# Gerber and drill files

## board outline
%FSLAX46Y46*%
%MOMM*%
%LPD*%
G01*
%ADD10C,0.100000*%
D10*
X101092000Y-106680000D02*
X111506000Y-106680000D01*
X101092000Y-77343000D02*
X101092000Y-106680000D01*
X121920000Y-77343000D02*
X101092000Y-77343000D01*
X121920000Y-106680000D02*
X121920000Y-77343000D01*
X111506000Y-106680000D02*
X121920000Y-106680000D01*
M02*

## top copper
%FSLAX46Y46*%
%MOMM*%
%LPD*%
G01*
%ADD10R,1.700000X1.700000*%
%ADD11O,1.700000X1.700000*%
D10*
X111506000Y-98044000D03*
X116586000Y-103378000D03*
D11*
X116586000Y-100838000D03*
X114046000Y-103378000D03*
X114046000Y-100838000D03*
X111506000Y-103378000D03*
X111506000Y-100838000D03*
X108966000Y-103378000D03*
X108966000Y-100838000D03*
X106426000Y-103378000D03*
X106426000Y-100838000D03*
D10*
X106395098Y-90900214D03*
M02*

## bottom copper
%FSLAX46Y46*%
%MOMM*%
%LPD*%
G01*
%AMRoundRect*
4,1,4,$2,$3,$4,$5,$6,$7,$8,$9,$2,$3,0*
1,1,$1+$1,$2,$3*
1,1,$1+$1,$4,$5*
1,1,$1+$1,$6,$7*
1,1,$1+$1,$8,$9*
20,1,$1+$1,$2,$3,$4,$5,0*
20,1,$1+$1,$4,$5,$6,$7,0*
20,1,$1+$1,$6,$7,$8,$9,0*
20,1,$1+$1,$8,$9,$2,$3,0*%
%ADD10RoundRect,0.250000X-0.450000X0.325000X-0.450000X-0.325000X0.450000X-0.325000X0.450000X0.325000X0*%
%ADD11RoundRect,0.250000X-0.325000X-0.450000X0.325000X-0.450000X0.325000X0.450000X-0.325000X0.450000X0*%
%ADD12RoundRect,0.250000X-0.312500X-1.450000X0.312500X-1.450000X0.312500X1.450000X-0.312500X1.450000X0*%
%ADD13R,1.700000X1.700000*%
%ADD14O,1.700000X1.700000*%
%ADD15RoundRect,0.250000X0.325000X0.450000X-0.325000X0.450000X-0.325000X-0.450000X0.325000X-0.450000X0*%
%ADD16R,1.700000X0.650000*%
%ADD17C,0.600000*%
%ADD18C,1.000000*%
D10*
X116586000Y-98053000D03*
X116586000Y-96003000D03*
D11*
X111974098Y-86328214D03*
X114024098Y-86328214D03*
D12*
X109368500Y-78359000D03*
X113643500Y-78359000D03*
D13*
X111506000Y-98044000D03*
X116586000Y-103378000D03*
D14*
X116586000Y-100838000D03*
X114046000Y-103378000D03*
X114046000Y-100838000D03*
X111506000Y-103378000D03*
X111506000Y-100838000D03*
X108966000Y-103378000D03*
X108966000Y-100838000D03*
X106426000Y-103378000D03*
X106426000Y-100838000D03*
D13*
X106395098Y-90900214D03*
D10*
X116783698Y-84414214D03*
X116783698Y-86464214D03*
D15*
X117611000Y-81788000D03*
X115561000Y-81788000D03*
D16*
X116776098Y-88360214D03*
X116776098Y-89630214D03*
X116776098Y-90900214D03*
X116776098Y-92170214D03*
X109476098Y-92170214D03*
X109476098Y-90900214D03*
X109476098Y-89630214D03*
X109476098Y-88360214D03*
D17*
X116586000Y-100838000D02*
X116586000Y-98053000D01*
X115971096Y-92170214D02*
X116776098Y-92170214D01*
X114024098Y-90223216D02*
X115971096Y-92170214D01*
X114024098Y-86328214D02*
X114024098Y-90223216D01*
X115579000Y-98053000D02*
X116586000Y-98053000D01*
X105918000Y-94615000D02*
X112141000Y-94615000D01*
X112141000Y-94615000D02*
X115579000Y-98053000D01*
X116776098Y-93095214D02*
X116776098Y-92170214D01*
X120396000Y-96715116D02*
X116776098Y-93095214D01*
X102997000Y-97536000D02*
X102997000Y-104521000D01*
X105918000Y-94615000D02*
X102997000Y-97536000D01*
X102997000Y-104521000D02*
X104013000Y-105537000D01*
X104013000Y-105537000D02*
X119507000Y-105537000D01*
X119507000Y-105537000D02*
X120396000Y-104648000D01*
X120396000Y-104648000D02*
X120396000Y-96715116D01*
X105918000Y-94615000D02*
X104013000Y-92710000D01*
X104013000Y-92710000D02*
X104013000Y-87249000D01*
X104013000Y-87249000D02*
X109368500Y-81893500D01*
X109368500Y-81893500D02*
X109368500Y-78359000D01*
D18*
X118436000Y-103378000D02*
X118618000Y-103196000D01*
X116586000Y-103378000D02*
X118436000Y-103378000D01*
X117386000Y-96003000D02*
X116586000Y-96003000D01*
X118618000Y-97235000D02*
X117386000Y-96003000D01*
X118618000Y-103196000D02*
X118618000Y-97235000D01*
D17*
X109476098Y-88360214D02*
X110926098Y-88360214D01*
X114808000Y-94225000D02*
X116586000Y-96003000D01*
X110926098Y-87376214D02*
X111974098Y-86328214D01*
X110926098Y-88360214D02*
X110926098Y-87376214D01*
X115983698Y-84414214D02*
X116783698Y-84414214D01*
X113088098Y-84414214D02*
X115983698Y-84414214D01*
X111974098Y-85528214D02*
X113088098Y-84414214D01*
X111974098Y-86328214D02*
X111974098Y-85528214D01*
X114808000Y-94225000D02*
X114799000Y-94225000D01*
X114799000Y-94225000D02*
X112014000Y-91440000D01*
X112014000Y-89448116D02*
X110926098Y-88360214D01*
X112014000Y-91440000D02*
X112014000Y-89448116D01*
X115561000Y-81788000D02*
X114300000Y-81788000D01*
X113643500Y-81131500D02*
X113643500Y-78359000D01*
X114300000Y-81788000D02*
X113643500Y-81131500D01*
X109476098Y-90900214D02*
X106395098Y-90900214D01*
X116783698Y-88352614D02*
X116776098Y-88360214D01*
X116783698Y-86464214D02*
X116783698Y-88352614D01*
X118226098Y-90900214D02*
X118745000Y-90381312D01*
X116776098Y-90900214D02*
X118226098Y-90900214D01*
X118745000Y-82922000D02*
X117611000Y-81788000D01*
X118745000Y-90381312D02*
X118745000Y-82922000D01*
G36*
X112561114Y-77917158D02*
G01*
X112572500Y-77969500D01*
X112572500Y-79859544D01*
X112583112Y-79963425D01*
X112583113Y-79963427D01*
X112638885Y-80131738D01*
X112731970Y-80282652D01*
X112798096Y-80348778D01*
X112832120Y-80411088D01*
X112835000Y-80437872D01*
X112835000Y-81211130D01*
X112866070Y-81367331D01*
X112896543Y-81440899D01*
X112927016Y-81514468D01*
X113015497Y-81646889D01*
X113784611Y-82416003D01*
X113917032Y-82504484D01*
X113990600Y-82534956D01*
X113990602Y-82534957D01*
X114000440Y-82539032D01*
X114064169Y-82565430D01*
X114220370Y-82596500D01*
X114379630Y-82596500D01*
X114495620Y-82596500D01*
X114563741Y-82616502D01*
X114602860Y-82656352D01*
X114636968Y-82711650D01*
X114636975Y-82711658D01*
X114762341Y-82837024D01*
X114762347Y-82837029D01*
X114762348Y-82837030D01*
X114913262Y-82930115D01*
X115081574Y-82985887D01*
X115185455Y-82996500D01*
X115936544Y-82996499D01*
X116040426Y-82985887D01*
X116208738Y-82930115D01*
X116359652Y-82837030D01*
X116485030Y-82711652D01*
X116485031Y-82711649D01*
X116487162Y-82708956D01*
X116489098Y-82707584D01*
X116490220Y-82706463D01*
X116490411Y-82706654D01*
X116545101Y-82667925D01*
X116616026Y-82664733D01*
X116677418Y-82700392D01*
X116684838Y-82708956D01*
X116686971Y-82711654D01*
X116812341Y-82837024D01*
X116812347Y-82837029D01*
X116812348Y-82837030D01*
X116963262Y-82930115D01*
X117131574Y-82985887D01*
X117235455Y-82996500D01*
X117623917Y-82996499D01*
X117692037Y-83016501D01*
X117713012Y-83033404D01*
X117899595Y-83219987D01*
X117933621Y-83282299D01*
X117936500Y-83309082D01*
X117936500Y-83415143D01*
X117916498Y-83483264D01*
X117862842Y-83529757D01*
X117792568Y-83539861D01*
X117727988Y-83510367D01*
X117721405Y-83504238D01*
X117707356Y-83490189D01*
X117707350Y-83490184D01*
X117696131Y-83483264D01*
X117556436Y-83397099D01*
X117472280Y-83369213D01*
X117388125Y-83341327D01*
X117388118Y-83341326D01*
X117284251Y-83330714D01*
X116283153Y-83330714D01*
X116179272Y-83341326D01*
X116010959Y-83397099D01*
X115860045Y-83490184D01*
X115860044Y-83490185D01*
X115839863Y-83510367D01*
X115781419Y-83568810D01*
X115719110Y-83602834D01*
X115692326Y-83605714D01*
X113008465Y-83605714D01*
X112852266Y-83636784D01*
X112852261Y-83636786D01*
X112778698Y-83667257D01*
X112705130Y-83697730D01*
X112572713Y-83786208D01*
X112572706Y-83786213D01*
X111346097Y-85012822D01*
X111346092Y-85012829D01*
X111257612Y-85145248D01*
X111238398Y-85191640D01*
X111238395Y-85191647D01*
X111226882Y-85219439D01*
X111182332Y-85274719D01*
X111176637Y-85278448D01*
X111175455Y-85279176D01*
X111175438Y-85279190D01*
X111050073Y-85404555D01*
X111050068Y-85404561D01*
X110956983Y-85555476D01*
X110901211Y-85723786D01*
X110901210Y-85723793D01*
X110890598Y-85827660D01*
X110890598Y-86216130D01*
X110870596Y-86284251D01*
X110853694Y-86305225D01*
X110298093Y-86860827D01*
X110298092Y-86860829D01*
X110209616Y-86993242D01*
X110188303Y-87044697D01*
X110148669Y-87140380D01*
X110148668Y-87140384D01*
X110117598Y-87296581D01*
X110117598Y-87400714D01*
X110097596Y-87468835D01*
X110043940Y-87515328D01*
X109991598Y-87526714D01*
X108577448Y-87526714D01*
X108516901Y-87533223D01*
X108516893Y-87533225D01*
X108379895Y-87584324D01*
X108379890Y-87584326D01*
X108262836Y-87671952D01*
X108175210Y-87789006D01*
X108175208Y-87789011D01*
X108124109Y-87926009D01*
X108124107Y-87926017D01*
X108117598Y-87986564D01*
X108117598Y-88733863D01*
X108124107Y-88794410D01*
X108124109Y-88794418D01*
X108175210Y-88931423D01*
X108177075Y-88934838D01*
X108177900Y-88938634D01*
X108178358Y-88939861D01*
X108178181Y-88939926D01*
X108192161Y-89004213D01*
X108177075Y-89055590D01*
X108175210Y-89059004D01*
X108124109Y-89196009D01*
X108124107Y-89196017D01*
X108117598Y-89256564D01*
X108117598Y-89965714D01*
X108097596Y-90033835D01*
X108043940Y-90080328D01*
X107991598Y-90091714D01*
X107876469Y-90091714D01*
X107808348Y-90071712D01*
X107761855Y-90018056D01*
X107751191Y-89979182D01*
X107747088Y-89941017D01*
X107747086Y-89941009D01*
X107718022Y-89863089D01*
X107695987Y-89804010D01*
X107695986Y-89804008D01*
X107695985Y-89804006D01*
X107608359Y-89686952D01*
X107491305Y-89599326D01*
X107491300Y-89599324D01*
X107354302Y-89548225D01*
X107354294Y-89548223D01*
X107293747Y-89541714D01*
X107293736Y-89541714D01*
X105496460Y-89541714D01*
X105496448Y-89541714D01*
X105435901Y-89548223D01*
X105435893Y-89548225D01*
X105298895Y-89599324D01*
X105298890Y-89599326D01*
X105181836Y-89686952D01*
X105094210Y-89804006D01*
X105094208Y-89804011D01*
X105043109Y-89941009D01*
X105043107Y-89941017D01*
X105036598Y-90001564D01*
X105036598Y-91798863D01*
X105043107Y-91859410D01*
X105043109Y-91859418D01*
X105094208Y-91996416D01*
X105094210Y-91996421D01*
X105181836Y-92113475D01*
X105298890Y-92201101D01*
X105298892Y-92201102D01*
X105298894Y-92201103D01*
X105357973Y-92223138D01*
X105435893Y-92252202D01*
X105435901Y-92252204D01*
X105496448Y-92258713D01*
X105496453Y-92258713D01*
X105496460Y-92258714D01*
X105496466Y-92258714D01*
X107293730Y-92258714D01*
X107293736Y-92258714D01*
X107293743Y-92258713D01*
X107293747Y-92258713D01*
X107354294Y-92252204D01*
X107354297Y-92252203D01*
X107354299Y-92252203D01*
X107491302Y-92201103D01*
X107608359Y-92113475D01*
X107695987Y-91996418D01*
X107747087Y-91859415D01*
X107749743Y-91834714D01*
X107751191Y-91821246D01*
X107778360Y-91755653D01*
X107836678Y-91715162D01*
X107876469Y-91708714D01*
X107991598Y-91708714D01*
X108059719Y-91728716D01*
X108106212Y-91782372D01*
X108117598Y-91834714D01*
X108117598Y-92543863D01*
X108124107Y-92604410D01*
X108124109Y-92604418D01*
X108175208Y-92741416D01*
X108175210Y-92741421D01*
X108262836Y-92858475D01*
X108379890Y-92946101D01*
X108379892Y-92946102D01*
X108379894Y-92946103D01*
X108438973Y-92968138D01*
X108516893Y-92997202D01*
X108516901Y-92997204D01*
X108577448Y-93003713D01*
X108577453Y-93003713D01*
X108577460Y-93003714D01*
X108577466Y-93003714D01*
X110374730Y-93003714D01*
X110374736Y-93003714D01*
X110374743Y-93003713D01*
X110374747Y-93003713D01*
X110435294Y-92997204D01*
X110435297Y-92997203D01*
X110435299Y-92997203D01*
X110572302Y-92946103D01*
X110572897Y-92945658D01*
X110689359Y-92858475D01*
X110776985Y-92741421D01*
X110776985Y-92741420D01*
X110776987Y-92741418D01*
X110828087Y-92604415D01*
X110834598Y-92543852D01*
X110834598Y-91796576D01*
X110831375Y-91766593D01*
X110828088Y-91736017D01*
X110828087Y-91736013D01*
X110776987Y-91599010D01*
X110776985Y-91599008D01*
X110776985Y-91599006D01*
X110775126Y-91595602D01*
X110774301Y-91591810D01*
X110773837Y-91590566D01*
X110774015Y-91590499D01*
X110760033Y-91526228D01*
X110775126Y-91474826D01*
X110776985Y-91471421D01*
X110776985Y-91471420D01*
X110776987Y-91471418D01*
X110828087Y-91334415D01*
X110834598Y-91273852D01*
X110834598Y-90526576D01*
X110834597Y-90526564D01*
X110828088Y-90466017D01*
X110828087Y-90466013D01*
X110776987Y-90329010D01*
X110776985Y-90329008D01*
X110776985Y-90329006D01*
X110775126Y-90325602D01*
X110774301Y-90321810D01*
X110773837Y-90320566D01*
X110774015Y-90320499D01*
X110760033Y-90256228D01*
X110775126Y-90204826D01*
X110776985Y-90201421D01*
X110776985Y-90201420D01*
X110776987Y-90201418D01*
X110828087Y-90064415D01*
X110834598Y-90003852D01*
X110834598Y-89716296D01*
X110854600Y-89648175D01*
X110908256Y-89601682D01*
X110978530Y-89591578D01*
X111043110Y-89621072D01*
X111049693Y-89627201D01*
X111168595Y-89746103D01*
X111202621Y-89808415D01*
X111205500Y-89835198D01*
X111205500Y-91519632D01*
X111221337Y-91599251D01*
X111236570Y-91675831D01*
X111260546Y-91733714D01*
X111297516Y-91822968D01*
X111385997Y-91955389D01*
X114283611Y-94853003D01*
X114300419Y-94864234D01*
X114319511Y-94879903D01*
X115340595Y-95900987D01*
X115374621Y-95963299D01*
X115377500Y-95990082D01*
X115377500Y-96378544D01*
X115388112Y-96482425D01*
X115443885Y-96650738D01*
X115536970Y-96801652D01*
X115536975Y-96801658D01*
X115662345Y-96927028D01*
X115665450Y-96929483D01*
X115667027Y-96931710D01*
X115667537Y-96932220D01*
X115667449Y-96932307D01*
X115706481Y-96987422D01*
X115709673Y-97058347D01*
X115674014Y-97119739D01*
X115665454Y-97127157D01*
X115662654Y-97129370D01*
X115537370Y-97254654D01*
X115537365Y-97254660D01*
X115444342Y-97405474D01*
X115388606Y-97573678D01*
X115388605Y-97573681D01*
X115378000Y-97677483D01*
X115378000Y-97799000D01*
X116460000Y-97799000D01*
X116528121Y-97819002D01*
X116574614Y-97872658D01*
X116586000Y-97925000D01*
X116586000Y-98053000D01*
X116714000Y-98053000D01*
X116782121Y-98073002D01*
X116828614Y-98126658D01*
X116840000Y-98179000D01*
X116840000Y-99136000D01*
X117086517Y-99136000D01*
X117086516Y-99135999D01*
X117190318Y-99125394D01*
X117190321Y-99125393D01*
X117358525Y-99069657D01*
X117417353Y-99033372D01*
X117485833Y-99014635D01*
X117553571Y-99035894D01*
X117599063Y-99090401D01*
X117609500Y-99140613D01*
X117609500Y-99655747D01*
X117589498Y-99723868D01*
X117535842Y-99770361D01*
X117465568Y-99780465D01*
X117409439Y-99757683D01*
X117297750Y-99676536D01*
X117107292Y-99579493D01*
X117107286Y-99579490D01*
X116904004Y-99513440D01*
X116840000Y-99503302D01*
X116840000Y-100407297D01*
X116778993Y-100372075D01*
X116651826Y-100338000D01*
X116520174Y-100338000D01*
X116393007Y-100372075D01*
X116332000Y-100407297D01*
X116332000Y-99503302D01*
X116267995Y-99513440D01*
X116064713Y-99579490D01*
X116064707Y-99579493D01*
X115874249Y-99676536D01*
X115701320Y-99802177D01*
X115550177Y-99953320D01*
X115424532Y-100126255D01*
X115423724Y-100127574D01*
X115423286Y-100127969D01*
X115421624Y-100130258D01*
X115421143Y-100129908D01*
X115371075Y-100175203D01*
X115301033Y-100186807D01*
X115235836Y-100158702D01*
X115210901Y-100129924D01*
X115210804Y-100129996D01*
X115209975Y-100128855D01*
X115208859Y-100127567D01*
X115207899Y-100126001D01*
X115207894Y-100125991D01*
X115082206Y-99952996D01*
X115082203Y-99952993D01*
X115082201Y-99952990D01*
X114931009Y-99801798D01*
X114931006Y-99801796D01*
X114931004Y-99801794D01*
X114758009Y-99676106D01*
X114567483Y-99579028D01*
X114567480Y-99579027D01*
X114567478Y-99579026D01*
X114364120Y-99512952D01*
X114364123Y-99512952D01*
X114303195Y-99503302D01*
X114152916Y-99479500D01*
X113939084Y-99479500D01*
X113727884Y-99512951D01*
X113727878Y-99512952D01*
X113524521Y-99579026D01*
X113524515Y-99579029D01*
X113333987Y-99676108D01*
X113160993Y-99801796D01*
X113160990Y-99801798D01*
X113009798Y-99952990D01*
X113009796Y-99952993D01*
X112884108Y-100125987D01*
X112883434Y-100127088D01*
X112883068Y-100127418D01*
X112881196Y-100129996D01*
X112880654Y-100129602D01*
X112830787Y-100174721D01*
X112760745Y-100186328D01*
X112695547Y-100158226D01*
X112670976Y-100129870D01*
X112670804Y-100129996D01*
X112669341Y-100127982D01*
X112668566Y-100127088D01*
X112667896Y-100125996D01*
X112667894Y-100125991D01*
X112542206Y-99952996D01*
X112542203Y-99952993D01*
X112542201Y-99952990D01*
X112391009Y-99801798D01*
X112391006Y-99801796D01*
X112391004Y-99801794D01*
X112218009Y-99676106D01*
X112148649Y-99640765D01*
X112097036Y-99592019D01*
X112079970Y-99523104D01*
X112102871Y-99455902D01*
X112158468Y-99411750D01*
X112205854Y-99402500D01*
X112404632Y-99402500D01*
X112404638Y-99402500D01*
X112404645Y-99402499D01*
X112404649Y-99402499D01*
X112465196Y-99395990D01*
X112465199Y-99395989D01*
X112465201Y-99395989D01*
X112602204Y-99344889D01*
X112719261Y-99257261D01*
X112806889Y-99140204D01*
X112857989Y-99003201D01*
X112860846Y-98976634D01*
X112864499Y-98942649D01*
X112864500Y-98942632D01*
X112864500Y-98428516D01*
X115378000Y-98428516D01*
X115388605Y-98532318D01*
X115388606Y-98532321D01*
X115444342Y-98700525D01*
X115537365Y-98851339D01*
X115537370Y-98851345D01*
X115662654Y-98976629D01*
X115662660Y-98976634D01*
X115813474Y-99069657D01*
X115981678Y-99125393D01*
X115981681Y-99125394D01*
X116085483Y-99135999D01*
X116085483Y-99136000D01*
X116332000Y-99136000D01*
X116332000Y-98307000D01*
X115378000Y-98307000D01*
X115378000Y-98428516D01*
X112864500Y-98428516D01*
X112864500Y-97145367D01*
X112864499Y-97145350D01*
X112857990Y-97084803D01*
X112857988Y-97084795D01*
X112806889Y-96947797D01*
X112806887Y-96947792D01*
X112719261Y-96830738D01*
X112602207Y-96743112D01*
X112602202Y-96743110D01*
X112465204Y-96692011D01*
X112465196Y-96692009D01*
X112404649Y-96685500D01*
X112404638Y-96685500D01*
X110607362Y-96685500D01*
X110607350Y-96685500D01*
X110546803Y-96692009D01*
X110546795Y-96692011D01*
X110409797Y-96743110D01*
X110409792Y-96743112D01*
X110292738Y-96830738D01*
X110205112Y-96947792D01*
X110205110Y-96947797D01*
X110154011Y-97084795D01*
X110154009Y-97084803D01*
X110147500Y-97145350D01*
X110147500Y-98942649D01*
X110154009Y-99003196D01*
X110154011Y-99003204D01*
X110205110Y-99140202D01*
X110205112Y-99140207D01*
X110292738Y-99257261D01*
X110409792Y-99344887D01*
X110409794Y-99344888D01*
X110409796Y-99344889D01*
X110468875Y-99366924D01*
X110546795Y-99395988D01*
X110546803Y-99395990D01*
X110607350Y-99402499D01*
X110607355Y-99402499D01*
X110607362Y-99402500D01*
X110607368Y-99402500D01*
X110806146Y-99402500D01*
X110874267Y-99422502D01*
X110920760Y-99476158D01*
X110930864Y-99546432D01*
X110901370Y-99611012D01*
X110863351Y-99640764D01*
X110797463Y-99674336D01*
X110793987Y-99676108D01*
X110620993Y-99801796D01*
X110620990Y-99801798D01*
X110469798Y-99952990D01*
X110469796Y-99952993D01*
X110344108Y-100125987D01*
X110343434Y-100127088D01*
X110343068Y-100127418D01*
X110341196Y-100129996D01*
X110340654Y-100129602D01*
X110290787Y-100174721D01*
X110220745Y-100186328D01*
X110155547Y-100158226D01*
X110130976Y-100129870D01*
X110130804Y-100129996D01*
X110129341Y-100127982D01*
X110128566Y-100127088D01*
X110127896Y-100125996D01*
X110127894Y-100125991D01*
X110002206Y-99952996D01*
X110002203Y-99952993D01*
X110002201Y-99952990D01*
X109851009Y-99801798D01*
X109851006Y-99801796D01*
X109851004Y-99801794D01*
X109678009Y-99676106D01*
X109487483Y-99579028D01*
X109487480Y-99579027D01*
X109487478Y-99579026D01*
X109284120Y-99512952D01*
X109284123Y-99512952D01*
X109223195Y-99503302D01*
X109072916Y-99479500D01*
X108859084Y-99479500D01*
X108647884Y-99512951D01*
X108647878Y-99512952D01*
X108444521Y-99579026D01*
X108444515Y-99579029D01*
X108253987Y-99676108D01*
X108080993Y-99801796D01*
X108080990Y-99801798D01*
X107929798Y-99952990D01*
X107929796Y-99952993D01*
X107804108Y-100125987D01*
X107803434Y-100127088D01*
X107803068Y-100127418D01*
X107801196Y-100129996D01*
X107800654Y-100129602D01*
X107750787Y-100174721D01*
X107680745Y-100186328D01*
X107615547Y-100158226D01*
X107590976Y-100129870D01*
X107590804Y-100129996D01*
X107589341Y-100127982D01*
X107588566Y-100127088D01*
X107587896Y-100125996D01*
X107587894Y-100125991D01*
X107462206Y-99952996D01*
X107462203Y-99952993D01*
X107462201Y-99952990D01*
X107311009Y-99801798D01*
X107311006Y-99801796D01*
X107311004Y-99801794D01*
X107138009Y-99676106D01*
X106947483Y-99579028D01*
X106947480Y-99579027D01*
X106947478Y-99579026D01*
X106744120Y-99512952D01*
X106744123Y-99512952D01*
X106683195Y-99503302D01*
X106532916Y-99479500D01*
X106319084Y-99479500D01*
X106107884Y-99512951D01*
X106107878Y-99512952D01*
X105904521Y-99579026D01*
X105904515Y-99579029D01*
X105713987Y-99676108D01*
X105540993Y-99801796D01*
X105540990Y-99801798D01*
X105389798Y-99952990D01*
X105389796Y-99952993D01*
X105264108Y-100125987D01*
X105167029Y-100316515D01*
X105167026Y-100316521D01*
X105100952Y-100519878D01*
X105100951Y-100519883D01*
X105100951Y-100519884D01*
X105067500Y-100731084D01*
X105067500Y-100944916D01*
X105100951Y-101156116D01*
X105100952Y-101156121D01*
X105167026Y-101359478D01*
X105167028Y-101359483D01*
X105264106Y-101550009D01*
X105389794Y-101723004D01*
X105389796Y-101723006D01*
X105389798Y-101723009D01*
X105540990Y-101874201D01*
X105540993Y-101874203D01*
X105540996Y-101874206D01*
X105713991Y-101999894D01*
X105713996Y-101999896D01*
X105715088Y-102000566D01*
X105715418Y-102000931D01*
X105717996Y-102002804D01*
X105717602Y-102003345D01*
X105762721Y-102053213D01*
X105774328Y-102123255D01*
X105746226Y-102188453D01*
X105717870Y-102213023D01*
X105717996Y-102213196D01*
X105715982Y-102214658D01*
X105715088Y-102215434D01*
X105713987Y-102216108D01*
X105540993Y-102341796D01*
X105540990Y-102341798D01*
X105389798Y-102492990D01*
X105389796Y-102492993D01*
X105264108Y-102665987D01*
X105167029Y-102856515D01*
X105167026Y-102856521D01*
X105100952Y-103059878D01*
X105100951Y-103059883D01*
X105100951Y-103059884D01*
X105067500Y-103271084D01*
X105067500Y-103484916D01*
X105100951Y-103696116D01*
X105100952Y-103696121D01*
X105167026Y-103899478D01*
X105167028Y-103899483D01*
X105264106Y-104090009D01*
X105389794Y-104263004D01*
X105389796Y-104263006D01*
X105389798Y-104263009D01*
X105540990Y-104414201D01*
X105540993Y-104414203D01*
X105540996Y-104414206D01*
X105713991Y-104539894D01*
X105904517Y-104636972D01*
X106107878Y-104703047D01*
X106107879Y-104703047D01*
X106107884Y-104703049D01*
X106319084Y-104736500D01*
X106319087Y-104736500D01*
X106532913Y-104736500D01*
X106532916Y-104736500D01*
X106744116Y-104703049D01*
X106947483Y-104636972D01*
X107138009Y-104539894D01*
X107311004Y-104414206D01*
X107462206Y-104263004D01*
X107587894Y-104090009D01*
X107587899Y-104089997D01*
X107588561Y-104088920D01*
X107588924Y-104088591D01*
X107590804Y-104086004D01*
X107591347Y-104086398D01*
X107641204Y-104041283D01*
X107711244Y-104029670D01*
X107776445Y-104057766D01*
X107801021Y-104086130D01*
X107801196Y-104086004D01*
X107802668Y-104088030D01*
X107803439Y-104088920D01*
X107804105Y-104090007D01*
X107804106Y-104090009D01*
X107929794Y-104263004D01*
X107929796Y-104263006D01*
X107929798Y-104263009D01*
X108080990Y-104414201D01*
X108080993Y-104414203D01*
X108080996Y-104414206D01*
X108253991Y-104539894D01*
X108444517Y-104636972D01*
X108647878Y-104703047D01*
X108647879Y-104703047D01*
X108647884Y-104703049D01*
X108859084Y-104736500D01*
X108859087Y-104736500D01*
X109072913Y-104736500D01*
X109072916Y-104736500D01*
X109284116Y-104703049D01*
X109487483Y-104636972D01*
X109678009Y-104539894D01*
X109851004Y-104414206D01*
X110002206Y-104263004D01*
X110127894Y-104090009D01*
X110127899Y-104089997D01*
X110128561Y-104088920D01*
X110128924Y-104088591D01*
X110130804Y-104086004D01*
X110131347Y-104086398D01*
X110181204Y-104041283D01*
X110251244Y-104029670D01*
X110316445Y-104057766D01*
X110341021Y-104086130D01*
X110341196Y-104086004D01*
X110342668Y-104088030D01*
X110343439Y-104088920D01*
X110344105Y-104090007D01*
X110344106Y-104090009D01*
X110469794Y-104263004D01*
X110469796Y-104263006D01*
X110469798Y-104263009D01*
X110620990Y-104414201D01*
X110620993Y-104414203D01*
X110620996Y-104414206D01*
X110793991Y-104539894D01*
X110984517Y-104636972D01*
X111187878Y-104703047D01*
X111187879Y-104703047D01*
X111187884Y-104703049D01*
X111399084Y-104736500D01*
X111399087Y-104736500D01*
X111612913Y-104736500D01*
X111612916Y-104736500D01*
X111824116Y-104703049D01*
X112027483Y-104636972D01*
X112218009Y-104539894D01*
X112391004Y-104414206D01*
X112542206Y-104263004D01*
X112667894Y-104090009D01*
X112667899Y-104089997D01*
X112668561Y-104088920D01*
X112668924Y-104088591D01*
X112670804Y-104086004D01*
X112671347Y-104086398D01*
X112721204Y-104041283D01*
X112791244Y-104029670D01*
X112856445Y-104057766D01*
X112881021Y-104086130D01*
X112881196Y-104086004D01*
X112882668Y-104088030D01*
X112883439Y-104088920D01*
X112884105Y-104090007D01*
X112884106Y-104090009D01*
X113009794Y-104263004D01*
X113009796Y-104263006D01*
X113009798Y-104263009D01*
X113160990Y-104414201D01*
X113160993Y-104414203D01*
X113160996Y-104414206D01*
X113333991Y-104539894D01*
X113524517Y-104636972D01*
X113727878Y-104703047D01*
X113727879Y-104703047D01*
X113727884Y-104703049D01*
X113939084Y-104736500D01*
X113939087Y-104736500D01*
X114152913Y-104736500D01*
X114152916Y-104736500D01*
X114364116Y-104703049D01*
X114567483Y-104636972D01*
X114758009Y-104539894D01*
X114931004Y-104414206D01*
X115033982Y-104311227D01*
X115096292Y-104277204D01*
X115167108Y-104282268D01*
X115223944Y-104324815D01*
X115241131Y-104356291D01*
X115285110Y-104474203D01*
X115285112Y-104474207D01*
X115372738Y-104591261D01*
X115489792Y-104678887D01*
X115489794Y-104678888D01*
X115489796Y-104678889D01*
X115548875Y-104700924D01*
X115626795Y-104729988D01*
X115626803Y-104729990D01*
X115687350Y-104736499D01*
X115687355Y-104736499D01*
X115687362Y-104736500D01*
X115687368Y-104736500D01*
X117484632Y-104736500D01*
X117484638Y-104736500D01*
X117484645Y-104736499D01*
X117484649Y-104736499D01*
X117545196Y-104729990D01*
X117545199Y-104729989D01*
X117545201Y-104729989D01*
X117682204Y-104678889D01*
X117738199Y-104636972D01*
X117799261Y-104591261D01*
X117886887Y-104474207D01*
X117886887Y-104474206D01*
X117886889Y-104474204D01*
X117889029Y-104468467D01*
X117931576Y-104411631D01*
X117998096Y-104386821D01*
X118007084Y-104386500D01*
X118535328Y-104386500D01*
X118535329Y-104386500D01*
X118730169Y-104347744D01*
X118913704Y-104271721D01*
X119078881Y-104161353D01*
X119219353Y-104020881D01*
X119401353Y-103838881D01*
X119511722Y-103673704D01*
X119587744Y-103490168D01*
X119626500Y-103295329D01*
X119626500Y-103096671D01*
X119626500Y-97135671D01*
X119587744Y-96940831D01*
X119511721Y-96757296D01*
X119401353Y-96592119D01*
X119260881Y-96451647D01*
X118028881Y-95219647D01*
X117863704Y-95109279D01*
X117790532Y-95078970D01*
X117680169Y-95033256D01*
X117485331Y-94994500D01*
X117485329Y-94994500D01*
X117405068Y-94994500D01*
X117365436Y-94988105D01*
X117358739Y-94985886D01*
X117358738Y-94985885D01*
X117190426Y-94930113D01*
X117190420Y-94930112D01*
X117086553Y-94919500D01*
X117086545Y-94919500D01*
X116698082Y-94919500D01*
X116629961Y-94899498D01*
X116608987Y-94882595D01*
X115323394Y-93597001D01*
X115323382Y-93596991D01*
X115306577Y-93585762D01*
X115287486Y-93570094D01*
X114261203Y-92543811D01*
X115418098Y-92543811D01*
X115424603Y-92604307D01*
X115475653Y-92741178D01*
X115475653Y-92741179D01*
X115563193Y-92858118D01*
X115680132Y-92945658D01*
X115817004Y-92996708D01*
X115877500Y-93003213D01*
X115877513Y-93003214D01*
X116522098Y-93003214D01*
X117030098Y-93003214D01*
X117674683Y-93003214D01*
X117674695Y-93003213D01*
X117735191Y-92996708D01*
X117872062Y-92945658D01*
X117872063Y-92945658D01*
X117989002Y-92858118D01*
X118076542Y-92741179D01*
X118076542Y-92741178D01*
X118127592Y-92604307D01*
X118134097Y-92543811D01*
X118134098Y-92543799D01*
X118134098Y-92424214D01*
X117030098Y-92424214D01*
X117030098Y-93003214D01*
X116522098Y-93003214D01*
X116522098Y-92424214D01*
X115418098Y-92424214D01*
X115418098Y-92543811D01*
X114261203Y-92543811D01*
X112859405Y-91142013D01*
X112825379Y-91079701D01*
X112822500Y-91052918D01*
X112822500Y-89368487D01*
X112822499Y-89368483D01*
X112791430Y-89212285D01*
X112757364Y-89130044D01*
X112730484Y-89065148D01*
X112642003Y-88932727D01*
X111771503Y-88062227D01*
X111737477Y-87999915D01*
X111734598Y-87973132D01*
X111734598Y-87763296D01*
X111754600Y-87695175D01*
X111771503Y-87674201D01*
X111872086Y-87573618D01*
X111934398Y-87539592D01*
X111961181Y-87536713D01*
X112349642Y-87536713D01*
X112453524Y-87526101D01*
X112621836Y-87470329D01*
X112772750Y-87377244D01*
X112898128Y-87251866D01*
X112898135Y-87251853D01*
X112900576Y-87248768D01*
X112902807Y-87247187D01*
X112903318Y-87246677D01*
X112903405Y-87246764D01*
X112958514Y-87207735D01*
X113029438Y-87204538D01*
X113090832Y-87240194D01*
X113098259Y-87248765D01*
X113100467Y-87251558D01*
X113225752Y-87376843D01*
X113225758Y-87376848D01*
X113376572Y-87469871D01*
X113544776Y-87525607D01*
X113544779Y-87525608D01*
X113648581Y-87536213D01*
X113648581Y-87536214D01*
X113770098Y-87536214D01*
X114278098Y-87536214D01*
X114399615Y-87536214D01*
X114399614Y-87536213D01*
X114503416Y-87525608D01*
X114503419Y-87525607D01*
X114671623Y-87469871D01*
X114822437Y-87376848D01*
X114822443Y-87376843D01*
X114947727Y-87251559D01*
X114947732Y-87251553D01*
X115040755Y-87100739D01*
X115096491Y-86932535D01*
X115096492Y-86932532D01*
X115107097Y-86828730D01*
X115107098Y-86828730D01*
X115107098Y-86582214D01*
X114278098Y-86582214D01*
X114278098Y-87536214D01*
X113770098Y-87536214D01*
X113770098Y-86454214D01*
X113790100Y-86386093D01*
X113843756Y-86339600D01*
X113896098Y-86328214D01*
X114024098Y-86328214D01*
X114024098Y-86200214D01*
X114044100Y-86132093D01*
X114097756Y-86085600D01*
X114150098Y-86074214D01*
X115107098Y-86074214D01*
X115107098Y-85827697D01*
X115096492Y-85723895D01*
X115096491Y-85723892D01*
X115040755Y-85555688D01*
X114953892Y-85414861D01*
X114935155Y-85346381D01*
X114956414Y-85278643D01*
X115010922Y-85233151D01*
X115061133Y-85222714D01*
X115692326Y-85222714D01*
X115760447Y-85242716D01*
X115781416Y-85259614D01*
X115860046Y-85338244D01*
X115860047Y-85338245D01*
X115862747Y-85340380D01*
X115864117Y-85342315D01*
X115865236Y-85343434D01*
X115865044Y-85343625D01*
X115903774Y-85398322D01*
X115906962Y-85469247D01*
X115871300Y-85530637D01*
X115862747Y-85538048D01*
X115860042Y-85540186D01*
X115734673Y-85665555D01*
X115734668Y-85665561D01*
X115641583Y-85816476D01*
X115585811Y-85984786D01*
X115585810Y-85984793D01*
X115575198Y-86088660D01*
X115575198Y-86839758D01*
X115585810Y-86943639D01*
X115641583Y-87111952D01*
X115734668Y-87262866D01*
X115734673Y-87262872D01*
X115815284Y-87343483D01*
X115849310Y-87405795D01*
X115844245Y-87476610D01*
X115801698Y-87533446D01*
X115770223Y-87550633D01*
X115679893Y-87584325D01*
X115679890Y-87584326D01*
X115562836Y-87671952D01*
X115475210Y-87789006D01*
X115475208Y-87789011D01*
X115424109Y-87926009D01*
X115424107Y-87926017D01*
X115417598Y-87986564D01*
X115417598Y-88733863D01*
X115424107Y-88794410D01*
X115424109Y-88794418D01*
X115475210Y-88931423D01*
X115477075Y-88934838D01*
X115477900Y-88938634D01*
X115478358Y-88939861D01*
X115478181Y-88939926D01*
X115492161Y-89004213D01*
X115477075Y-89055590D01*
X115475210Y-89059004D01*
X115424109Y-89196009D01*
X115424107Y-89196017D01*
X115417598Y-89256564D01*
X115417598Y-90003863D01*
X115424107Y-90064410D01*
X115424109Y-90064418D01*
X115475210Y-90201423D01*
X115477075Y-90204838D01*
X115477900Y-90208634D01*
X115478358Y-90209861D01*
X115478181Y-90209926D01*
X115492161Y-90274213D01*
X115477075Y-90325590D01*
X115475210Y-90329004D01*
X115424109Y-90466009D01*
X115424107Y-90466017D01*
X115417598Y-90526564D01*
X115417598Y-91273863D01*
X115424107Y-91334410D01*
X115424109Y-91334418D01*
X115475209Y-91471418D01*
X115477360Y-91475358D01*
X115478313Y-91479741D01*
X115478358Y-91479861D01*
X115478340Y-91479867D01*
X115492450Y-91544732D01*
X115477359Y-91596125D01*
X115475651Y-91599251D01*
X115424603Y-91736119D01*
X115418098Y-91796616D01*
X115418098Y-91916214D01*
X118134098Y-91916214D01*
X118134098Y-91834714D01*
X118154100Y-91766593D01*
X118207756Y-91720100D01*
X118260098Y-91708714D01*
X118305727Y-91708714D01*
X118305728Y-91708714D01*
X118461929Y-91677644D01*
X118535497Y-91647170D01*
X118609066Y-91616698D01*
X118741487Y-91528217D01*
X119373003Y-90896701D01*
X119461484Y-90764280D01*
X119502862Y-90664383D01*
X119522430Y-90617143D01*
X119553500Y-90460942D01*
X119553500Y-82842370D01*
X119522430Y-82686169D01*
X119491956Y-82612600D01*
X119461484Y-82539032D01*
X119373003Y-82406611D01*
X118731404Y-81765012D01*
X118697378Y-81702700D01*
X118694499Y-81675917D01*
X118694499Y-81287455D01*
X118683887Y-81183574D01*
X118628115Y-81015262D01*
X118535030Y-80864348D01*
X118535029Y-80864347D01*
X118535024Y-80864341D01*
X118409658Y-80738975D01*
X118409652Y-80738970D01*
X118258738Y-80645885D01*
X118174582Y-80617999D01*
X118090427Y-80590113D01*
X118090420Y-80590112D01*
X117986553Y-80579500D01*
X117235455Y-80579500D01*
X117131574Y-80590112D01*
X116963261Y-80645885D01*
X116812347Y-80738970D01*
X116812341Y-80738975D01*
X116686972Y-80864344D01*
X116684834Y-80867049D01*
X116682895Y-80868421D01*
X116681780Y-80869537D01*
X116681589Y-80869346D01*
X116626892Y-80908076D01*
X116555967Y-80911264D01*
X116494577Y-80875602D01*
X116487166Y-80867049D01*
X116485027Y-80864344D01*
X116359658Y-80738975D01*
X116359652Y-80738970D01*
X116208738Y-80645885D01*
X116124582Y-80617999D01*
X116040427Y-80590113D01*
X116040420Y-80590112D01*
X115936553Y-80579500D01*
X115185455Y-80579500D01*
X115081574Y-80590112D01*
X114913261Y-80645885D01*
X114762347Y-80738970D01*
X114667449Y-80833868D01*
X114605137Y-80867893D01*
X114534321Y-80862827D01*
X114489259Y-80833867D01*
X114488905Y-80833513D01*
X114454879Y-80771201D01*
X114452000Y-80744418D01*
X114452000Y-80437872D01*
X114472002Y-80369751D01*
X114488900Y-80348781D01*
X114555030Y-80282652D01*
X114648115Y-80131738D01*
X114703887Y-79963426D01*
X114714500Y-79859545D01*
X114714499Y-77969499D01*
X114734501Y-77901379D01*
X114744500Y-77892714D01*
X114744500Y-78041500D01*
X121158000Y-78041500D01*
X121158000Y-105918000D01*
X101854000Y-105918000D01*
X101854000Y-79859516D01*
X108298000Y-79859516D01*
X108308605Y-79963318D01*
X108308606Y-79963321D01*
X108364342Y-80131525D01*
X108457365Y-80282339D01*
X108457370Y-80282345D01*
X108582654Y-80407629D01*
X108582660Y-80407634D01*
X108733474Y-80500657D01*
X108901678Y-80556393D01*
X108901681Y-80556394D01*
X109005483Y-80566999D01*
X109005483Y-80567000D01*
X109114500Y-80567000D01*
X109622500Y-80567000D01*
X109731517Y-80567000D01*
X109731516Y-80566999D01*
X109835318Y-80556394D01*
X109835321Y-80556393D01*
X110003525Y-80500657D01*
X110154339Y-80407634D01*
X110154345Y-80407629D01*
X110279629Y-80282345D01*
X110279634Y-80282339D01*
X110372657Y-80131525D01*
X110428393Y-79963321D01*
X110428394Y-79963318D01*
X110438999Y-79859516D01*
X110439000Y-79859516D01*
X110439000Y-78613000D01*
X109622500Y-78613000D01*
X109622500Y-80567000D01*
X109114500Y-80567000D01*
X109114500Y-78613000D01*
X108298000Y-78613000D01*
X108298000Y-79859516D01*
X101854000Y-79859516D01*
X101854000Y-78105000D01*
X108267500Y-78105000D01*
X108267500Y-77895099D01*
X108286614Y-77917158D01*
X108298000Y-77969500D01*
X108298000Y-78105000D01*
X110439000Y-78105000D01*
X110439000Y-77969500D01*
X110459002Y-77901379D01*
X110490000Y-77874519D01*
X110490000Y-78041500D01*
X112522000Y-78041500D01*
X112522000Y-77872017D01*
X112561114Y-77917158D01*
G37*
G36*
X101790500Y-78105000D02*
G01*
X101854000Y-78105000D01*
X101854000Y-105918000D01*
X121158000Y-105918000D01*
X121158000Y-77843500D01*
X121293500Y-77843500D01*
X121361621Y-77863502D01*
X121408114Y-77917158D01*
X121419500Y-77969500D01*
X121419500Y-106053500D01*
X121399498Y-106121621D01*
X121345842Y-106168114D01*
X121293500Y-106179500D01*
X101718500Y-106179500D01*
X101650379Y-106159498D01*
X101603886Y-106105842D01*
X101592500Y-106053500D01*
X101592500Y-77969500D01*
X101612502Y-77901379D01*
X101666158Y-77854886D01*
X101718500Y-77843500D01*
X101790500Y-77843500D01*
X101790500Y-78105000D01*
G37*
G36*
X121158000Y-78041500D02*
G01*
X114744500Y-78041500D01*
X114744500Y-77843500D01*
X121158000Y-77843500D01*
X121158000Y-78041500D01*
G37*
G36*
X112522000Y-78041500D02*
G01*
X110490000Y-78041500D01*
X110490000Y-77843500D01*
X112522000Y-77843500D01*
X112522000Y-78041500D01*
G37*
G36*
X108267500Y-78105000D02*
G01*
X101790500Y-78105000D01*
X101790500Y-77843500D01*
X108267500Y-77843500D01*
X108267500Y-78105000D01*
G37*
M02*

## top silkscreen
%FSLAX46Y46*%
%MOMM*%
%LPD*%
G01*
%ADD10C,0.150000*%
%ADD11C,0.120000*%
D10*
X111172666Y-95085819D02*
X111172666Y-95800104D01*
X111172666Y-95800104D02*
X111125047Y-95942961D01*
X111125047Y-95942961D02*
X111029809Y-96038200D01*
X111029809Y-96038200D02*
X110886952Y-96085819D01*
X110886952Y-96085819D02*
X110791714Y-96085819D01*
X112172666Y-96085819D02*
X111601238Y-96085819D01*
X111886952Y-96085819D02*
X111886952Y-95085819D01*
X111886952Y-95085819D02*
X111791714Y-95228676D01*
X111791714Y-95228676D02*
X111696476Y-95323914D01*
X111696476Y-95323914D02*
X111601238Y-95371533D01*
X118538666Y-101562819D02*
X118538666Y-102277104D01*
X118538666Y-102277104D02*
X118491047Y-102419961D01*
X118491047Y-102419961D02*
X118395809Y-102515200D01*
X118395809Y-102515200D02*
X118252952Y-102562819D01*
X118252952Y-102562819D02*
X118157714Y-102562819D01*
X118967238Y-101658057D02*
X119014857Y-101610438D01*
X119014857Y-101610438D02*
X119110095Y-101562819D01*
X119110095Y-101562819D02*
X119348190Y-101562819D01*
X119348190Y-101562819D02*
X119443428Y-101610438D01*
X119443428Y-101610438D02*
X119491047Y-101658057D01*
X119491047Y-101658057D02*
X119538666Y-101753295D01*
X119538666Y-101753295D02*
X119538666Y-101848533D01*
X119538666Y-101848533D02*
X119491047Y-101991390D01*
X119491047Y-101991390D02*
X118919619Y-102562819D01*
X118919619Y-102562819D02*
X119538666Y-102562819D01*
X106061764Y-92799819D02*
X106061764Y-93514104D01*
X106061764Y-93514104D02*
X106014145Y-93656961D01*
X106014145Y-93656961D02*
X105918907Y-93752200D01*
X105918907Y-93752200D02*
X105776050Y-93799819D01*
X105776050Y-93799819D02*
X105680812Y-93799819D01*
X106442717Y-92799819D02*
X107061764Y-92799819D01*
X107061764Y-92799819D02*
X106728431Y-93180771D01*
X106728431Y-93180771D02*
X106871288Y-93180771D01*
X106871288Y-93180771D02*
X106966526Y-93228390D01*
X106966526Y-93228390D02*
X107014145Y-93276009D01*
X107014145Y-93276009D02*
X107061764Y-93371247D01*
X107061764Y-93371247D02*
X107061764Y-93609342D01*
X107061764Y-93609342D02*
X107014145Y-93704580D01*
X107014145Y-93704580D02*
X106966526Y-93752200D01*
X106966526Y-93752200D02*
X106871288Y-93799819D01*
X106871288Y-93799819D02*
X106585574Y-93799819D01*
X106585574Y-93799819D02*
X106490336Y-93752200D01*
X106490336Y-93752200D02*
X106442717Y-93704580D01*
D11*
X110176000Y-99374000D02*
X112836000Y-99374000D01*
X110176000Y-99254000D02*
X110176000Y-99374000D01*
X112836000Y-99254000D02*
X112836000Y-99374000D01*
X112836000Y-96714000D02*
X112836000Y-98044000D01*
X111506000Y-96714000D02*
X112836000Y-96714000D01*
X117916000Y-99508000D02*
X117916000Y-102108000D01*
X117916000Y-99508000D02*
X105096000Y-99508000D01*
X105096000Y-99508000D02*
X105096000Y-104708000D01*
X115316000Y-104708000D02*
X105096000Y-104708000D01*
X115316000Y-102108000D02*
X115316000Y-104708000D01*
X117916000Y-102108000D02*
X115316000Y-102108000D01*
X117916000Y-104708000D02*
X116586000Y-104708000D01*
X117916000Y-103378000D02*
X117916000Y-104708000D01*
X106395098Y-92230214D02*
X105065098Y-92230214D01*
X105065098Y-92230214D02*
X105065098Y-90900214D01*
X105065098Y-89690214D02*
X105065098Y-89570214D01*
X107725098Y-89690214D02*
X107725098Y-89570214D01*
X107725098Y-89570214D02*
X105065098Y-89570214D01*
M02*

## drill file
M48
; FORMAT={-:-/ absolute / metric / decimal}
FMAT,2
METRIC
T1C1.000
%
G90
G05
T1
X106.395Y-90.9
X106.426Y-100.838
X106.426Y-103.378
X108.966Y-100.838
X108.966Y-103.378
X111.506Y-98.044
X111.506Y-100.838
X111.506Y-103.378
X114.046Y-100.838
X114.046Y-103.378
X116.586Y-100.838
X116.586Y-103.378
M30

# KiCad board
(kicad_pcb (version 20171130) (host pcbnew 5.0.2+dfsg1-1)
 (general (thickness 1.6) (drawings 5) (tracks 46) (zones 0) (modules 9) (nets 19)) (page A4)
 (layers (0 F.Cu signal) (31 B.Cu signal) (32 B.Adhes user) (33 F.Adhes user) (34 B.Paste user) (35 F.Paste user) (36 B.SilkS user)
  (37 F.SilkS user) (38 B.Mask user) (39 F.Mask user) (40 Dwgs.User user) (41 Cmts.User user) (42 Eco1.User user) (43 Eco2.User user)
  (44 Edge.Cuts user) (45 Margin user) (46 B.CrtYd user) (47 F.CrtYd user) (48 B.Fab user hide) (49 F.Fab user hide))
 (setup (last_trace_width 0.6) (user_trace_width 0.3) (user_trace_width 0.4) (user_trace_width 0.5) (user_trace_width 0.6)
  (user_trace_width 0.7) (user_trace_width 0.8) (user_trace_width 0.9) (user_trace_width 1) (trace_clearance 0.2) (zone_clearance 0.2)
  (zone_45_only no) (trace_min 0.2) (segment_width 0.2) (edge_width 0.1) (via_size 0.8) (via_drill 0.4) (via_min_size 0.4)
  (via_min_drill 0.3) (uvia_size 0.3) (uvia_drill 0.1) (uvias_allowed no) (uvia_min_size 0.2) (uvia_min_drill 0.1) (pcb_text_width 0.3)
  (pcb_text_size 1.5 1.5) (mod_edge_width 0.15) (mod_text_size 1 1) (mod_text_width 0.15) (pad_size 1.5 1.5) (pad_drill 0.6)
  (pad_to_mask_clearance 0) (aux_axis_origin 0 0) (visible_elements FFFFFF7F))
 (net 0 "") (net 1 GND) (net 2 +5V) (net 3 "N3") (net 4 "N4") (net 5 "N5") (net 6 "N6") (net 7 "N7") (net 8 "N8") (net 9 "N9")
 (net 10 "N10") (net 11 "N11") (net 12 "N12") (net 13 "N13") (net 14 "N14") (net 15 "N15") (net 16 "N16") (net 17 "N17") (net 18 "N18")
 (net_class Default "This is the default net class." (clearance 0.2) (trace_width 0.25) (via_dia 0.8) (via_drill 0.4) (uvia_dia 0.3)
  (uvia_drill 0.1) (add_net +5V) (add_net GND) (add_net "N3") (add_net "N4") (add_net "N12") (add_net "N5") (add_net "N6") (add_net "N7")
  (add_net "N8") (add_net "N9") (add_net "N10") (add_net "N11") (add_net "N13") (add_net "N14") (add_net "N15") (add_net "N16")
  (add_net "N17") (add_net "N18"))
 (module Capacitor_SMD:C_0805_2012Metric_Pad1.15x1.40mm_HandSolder (layer B.Cu) (at 116.586 97.028 270)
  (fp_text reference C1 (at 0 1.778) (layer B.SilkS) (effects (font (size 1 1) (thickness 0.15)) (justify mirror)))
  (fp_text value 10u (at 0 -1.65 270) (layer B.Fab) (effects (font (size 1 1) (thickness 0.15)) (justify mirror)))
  (pad 2 smd roundrect (at 1.025 0 270) (size 1.15 1.4) (layers B.Cu B.Paste B.Mask) (roundrect_rratio 0.217391) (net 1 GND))
  (pad 1 smd roundrect (at -1.025 0 270) (size 1.15 1.4) (layers B.Cu B.Paste B.Mask) (roundrect_rratio 0.217391) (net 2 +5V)))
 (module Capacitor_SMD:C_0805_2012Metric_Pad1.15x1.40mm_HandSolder (layer B.Cu) (at 112.999098 86.328214)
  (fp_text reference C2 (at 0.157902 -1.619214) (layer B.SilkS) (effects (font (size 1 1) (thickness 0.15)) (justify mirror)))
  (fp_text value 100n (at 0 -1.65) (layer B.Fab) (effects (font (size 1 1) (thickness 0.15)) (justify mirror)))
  (pad 1 smd roundrect (at -1.025 0) (size 1.15 1.4) (layers B.Cu B.Paste B.Mask) (roundrect_rratio 0.217391) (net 2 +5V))
  (pad 2 smd roundrect (at 1.025 0) (size 1.15 1.4) (layers B.Cu B.Paste B.Mask) (roundrect_rratio 0.217391) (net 1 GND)))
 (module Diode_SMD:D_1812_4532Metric (layer B.Cu) (at 111.506 78.359)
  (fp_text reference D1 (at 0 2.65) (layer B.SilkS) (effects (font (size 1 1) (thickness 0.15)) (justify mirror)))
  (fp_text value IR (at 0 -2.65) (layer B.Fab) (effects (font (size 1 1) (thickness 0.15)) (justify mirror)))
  (pad 1 smd roundrect (at -2.1375 0) (size 1.125 3.4) (layers B.Cu B.Paste B.Mask) (roundrect_rratio 0.222222) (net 1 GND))
  (pad 2 smd roundrect (at 2.1375 0) (size 1.125 3.4) (layers B.Cu B.Paste B.Mask) (roundrect_rratio 0.222222) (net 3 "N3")))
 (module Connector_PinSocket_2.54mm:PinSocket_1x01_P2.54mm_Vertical (layer F.Cu) (at 111.506 98.044)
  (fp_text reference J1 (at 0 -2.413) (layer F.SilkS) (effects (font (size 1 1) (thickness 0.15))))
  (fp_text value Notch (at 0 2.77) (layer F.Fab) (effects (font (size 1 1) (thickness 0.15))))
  (fp_line (start -1.33 1.33) (end 1.33 1.33) (layer F.SilkS) (width 0.12))
  (fp_line (start -1.33 1.21) (end -1.33 1.33) (layer F.SilkS) (width 0.12))
  (fp_line (start 1.33 1.21) (end 1.33 1.33) (layer F.SilkS) (width 0.12))
  (fp_line (start 1.33 -1.33) (end 1.33 0) (layer F.SilkS) (width 0.12))
  (fp_line (start 0 -1.33) (end 1.33 -1.33) (layer F.SilkS) (width 0.12))
  (pad 1 thru_hole rect (at 0 0) (size 1.7 1.7) (drill 1) (layers *.Cu *.Mask) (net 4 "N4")))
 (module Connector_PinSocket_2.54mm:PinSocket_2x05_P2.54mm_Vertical (layer F.Cu) (at 116.586 103.378 270)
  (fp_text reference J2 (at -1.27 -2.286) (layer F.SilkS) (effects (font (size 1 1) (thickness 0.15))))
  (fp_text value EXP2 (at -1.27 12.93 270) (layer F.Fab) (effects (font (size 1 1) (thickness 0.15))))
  (fp_line (start -3.87 -1.33) (end -1.27 -1.33) (layer F.SilkS) (width 0.12))
  (fp_line (start -3.87 -1.33) (end -3.87 11.49) (layer F.SilkS) (width 0.12))
  (fp_line (start -3.87 11.49) (end 1.33 11.49) (layer F.SilkS) (width 0.12))
  (fp_line (start 1.33 1.27) (end 1.33 11.49) (layer F.SilkS) (width 0.12))
  (fp_line (start -1.27 1.27) (end 1.33 1.27) (layer F.SilkS) (width 0.12))
  (fp_line (start -1.27 -1.33) (end -1.27 1.27) (layer F.SilkS) (width 0.12))
  (fp_line (start 1.33 -1.33) (end 1.33 0) (layer F.SilkS) (width 0.12))
  (fp_line (start 0 -1.33) (end 1.33 -1.33) (layer F.SilkS) (width 0.12))
  (pad 1 thru_hole rect (at 0 0 270) (size 1.7 1.7) (drill 1) (layers *.Cu *.Mask) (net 2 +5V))
  (pad 2 thru_hole oval (at -2.54 0 270) (size 1.7 1.7) (drill 1) (layers *.Cu *.Mask) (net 1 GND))
  (pad 3 thru_hole oval (at 0 2.54 270) (size 1.7 1.7) (drill 1) (layers *.Cu *.Mask) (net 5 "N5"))
  (pad 4 thru_hole oval (at -2.54 2.54 270) (size 1.7 1.7) (drill 1) (layers *.Cu *.Mask) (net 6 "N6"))
  (pad 5 thru_hole oval (at 0 5.08 270) (size 1.7 1.7) (drill 1) (layers *.Cu *.Mask) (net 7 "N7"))
  (pad 6 thru_hole oval (at -2.54 5.08 270) (size 1.7 1.7) (drill 1) (layers *.Cu *.Mask) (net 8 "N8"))
  (pad 7 thru_hole oval (at 0 7.62 270) (size 1.7 1.7) (drill 1) (layers *.Cu *.Mask) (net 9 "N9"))
  (pad 8 thru_hole oval (at -2.54 7.62 270) (size 1.7 1.7) (drill 1) (layers *.Cu *.Mask) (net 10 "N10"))
  (pad 9 thru_hole oval (at 0 10.16 270) (size 1.7 1.7) (drill 1) (layers *.Cu *.Mask) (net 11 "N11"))
  (pad 10 thru_hole oval (at -2.54 10.16 270) (size 1.7 1.7) (drill 1) (layers *.Cu *.Mask) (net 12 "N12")))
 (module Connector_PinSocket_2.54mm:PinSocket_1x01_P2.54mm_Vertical (layer F.Cu) (at 106.395098 90.900214 180)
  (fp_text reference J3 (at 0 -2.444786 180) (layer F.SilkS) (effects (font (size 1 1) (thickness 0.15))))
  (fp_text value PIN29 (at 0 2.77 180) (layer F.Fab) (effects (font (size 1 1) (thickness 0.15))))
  (fp_line (start 0 -1.33) (end 1.33 -1.33) (layer F.SilkS) (width 0.12))
  (fp_line (start 1.33 -1.33) (end 1.33 0) (layer F.SilkS) (width 0.12))
  (fp_line (start 1.33 1.21) (end 1.33 1.33) (layer F.SilkS) (width 0.12))
  (fp_line (start -1.33 1.21) (end -1.33 1.33) (layer F.SilkS) (width 0.12))
  (fp_line (start -1.33 1.33) (end 1.33 1.33) (layer F.SilkS) (width 0.12))
  (pad 1 thru_hole rect (at 0 0 180) (size 1.7 1.7) (drill 1) (layers *.Cu *.Mask) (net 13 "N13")))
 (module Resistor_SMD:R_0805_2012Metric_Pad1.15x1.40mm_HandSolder (layer B.Cu) (at 116.783698 85.439214 270)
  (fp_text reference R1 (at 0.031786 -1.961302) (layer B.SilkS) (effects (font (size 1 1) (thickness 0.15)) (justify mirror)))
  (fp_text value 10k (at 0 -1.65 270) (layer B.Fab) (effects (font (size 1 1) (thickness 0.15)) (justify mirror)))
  (pad 1 smd roundrect (at -1.025 0 270) (size 1.15 1.4) (layers B.Cu B.Paste B.Mask) (roundrect_rratio 0.217391) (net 2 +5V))
  (pad 2 smd roundrect (at 1.025 0 270) (size 1.15 1.4) (layers B.Cu B.Paste B.Mask) (roundrect_rratio 0.217391) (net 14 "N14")))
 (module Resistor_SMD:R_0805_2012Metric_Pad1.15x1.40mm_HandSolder (layer B.Cu) (at 116.586 81.788 180)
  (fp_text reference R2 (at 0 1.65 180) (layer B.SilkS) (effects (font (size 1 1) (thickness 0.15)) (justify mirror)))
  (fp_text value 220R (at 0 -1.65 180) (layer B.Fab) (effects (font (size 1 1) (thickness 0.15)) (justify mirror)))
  (pad 1 smd roundrect (at -1.025 0 180) (size 1.15 1.4) (layers B.Cu B.Paste B.Mask) (roundrect_rratio 0.217391) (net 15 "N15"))
  (pad 2 smd roundrect (at 1.025 0 180) (size 1.15 1.4) (layers B.Cu B.Paste B.Mask) (roundrect_rratio 0.217391) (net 3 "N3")))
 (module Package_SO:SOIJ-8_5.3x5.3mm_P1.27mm (layer B.Cu) (at 113.126098 90.265214 180)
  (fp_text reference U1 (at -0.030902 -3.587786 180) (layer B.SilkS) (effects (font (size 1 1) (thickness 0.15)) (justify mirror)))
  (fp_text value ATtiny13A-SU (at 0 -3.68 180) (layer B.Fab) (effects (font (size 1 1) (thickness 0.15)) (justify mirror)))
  (pad 1 smd rect (at -3.65 1.905 180) (size 1.7 0.65) (layers B.Cu B.Paste B.Mask) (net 14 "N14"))
  (pad 2 smd rect (at -3.65 0.635 180) (size 1.7 0.65) (layers B.Cu B.Paste B.Mask) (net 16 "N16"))
  (pad 3 smd rect (at -3.65 -0.635 180) (size 1.7 0.65) (layers B.Cu B.Paste B.Mask) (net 15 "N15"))
  (pad 4 smd rect (at -3.65 -1.905 180) (size 1.7 0.65) (layers B.Cu B.Paste B.Mask) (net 1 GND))
  (pad 5 smd rect (at 3.65 -1.905 180) (size 1.7 0.65) (layers B.Cu B.Paste B.Mask) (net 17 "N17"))
  (pad 6 smd rect (at 3.65 -0.635 180) (size 1.7 0.65) (layers B.Cu B.Paste B.Mask) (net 13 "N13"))
  (pad 7 smd rect (at 3.65 0.635 180) (size 1.7 0.65) (layers B.Cu B.Paste B.Mask) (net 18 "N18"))
  (pad 8 smd rect (at 3.65 1.905 180) (size 1.7 0.65) (layers B.Cu B.Paste B.Mask) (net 2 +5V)))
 (gr_line (start 101.092 106.68) (end 111.506 106.68) (layer Edge.Cuts) (width 0.1))
 (gr_line (start 101.092 77.343) (end 101.092 106.68) (layer Edge.Cuts) (width 0.1))
 (gr_line (start 121.92 77.343) (end 101.092 77.343) (layer Edge.Cuts) (width 0.1))
 (gr_line (start 121.92 106.68) (end 121.92 77.343) (layer Edge.Cuts) (width 0.1))
 (gr_line (start 111.506 106.68) (end 121.92 106.68) (layer Edge.Cuts) (width 0.1))
 (segment (start 116.586 100.838) (end 116.586 98.053) (width 0.6) (layer B.Cu) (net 1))
 (segment (start 115.971096 92.170214) (end 116.776098 92.170214) (width 0.6) (layer B.Cu) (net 1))
 (segment (start 114.024098 90.223216) (end 115.971096 92.170214) (width 0.6) (layer B.Cu) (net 1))
 (segment (start 114.024098 86.328214) (end 114.024098 90.223216) (width 0.6) (layer B.Cu) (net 1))
 (segment (start 115.579 98.053) (end 116.586 98.053) (width 0.6) (layer B.Cu) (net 1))
 (segment (start 105.918 94.615) (end 112.141 94.615) (width 0.6) (layer B.Cu) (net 1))
 (segment (start 112.141 94.615) (end 115.579 98.053) (width 0.6) (layer B.Cu) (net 1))
 (segment (start 116.776098 93.095214) (end 116.776098 92.170214) (width 0.6) (layer B.Cu) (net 1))
 (segment (start 120.396 96.715116) (end 116.776098 93.095214) (width 0.6) (layer B.Cu) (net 1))
 (segment (start 102.997 97.536) (end 102.997 104.521) (width 0.6) (layer B.Cu) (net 1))
 (segment (start 105.918 94.615) (end 102.997 97.536) (width 0.6) (layer B.Cu) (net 1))
 (segment (start 102.997 104.521) (end 104.013 105.537) (width 0.6) (layer B.Cu) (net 1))
 (segment (start 104.013 105.537) (end 119.507 105.537) (width 0.6) (layer B.Cu) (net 1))
 (segment (start 119.507 105.537) (end 120.396 104.648) (width 0.6) (layer B.Cu) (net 1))
 (segment (start 120.396 104.648) (end 120.396 96.715116) (width 0.6) (layer B.Cu) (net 1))
 (segment (start 105.918 94.615) (end 104.013 92.71) (width 0.6) (layer B.Cu) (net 1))
 (segment (start 104.013 92.71) (end 104.013 87.249) (width 0.6) (layer B.Cu) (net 1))
 (segment (start 104.013 87.249) (end 109.3685 81.8935) (width 0.6) (layer B.Cu) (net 1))
 (segment (start 109.3685 81.8935) (end 109.3685 78.359) (width 0.6) (layer B.Cu) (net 1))
 (segment (start 118.436 103.378) (end 118.618 103.196) (width 1) (layer B.Cu) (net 2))
 (segment (start 116.586 103.378) (end 118.436 103.378) (width 1) (layer B.Cu) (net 2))
 (segment (start 117.386 96.003) (end 116.586 96.003) (width 1) (layer B.Cu) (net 2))
 (segment (start 118.618 97.235) (end 117.386 96.003) (width 1) (layer B.Cu) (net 2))
 (segment (start 118.618 103.196) (end 118.618 97.235) (width 1) (layer B.Cu) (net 2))
 (segment (start 109.476098 88.360214) (end 110.926098 88.360214) (width 0.6) (layer B.Cu) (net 2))
 (segment (start 114.808 94.225) (end 116.586 96.003) (width 0.6) (layer B.Cu) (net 2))
 (segment (start 110.926098 87.376214) (end 111.974098 86.328214) (width 0.6) (layer B.Cu) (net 2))
 (segment (start 110.926098 88.360214) (end 110.926098 87.376214) (width 0.6) (layer B.Cu) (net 2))
 (segment (start 115.983698 84.414214) (end 116.783698 84.414214) (width 0.6) (layer B.Cu) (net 2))
 (segment (start 113.088098 84.414214) (end 115.983698 84.414214) (width 0.6) (layer B.Cu) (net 2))
 (segment (start 111.974098 85.528214) (end 113.088098 84.414214) (width 0.6) (layer B.Cu) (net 2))
 (segment (start 111.974098 86.328214) (end 111.974098 85.528214) (width 0.6) (layer B.Cu) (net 2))
 (segment (start 114.808 94.225) (end 114.799 94.225) (width 0.6) (layer B.Cu) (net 2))
 (segment (start 114.799 94.225) (end 112.014 91.44) (width 0.6) (layer B.Cu) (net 2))
 (segment (start 112.014 89.448116) (end 110.926098 88.360214) (width 0.6) (layer B.Cu) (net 2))
 (segment (start 112.014 91.44) (end 112.014 89.448116) (width 0.6) (layer B.Cu) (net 2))
 (segment (start 115.561 81.788) (end 114.3 81.788) (width 0.6) (layer B.Cu) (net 3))
 (segment (start 113.6435 81.1315) (end 113.6435 78.359) (width 0.6) (layer B.Cu) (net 3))
 (segment (start 114.3 81.788) (end 113.6435 81.1315) (width 0.6) (layer B.Cu) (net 3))
 (segment (start 109.476098 90.900214) (end 106.395098 90.900214) (width 0.6) (layer B.Cu) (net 13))
 (segment (start 116.783698 88.352614) (end 116.776098 88.360214) (width 0.6) (layer B.Cu) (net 14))
 (segment (start 116.783698 86.464214) (end 116.783698 88.352614) (width 0.6) (layer B.Cu) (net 14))
 (segment (start 118.226098 90.900214) (end 118.745 90.381312) (width 0.6) (layer B.Cu) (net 15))
 (segment (start 116.776098 90.900214) (end 118.226098 90.900214) (width 0.6) (layer B.Cu) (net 15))
 (segment (start 118.745 82.922) (end 117.611 81.788) (width 0.6) (layer B.Cu) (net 15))
 (segment (start 118.745 90.381312) (end 118.745 82.922) (width 0.6) (layer B.Cu) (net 15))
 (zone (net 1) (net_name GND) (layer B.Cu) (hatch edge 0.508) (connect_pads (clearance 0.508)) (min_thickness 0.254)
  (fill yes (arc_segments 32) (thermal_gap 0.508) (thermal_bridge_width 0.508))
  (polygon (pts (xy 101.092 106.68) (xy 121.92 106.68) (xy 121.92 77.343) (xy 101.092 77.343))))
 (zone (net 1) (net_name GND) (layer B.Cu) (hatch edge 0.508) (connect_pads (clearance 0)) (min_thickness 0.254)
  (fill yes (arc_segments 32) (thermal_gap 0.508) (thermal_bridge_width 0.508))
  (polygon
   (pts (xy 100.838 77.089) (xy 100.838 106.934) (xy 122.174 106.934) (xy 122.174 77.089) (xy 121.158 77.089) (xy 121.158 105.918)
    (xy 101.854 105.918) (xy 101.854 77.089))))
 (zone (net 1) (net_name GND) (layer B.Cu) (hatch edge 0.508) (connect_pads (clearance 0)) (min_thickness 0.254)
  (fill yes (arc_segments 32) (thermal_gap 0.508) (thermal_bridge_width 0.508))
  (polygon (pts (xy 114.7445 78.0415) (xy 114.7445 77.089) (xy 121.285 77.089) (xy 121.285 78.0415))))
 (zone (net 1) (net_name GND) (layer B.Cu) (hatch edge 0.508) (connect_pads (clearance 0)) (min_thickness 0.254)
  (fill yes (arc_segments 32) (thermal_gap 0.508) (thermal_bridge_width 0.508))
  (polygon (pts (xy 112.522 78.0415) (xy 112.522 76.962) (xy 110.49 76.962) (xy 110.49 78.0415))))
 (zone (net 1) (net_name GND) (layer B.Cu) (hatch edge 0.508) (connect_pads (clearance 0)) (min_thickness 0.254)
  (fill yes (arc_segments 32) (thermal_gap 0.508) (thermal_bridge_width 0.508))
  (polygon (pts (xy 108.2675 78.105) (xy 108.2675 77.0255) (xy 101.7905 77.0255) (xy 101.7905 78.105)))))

